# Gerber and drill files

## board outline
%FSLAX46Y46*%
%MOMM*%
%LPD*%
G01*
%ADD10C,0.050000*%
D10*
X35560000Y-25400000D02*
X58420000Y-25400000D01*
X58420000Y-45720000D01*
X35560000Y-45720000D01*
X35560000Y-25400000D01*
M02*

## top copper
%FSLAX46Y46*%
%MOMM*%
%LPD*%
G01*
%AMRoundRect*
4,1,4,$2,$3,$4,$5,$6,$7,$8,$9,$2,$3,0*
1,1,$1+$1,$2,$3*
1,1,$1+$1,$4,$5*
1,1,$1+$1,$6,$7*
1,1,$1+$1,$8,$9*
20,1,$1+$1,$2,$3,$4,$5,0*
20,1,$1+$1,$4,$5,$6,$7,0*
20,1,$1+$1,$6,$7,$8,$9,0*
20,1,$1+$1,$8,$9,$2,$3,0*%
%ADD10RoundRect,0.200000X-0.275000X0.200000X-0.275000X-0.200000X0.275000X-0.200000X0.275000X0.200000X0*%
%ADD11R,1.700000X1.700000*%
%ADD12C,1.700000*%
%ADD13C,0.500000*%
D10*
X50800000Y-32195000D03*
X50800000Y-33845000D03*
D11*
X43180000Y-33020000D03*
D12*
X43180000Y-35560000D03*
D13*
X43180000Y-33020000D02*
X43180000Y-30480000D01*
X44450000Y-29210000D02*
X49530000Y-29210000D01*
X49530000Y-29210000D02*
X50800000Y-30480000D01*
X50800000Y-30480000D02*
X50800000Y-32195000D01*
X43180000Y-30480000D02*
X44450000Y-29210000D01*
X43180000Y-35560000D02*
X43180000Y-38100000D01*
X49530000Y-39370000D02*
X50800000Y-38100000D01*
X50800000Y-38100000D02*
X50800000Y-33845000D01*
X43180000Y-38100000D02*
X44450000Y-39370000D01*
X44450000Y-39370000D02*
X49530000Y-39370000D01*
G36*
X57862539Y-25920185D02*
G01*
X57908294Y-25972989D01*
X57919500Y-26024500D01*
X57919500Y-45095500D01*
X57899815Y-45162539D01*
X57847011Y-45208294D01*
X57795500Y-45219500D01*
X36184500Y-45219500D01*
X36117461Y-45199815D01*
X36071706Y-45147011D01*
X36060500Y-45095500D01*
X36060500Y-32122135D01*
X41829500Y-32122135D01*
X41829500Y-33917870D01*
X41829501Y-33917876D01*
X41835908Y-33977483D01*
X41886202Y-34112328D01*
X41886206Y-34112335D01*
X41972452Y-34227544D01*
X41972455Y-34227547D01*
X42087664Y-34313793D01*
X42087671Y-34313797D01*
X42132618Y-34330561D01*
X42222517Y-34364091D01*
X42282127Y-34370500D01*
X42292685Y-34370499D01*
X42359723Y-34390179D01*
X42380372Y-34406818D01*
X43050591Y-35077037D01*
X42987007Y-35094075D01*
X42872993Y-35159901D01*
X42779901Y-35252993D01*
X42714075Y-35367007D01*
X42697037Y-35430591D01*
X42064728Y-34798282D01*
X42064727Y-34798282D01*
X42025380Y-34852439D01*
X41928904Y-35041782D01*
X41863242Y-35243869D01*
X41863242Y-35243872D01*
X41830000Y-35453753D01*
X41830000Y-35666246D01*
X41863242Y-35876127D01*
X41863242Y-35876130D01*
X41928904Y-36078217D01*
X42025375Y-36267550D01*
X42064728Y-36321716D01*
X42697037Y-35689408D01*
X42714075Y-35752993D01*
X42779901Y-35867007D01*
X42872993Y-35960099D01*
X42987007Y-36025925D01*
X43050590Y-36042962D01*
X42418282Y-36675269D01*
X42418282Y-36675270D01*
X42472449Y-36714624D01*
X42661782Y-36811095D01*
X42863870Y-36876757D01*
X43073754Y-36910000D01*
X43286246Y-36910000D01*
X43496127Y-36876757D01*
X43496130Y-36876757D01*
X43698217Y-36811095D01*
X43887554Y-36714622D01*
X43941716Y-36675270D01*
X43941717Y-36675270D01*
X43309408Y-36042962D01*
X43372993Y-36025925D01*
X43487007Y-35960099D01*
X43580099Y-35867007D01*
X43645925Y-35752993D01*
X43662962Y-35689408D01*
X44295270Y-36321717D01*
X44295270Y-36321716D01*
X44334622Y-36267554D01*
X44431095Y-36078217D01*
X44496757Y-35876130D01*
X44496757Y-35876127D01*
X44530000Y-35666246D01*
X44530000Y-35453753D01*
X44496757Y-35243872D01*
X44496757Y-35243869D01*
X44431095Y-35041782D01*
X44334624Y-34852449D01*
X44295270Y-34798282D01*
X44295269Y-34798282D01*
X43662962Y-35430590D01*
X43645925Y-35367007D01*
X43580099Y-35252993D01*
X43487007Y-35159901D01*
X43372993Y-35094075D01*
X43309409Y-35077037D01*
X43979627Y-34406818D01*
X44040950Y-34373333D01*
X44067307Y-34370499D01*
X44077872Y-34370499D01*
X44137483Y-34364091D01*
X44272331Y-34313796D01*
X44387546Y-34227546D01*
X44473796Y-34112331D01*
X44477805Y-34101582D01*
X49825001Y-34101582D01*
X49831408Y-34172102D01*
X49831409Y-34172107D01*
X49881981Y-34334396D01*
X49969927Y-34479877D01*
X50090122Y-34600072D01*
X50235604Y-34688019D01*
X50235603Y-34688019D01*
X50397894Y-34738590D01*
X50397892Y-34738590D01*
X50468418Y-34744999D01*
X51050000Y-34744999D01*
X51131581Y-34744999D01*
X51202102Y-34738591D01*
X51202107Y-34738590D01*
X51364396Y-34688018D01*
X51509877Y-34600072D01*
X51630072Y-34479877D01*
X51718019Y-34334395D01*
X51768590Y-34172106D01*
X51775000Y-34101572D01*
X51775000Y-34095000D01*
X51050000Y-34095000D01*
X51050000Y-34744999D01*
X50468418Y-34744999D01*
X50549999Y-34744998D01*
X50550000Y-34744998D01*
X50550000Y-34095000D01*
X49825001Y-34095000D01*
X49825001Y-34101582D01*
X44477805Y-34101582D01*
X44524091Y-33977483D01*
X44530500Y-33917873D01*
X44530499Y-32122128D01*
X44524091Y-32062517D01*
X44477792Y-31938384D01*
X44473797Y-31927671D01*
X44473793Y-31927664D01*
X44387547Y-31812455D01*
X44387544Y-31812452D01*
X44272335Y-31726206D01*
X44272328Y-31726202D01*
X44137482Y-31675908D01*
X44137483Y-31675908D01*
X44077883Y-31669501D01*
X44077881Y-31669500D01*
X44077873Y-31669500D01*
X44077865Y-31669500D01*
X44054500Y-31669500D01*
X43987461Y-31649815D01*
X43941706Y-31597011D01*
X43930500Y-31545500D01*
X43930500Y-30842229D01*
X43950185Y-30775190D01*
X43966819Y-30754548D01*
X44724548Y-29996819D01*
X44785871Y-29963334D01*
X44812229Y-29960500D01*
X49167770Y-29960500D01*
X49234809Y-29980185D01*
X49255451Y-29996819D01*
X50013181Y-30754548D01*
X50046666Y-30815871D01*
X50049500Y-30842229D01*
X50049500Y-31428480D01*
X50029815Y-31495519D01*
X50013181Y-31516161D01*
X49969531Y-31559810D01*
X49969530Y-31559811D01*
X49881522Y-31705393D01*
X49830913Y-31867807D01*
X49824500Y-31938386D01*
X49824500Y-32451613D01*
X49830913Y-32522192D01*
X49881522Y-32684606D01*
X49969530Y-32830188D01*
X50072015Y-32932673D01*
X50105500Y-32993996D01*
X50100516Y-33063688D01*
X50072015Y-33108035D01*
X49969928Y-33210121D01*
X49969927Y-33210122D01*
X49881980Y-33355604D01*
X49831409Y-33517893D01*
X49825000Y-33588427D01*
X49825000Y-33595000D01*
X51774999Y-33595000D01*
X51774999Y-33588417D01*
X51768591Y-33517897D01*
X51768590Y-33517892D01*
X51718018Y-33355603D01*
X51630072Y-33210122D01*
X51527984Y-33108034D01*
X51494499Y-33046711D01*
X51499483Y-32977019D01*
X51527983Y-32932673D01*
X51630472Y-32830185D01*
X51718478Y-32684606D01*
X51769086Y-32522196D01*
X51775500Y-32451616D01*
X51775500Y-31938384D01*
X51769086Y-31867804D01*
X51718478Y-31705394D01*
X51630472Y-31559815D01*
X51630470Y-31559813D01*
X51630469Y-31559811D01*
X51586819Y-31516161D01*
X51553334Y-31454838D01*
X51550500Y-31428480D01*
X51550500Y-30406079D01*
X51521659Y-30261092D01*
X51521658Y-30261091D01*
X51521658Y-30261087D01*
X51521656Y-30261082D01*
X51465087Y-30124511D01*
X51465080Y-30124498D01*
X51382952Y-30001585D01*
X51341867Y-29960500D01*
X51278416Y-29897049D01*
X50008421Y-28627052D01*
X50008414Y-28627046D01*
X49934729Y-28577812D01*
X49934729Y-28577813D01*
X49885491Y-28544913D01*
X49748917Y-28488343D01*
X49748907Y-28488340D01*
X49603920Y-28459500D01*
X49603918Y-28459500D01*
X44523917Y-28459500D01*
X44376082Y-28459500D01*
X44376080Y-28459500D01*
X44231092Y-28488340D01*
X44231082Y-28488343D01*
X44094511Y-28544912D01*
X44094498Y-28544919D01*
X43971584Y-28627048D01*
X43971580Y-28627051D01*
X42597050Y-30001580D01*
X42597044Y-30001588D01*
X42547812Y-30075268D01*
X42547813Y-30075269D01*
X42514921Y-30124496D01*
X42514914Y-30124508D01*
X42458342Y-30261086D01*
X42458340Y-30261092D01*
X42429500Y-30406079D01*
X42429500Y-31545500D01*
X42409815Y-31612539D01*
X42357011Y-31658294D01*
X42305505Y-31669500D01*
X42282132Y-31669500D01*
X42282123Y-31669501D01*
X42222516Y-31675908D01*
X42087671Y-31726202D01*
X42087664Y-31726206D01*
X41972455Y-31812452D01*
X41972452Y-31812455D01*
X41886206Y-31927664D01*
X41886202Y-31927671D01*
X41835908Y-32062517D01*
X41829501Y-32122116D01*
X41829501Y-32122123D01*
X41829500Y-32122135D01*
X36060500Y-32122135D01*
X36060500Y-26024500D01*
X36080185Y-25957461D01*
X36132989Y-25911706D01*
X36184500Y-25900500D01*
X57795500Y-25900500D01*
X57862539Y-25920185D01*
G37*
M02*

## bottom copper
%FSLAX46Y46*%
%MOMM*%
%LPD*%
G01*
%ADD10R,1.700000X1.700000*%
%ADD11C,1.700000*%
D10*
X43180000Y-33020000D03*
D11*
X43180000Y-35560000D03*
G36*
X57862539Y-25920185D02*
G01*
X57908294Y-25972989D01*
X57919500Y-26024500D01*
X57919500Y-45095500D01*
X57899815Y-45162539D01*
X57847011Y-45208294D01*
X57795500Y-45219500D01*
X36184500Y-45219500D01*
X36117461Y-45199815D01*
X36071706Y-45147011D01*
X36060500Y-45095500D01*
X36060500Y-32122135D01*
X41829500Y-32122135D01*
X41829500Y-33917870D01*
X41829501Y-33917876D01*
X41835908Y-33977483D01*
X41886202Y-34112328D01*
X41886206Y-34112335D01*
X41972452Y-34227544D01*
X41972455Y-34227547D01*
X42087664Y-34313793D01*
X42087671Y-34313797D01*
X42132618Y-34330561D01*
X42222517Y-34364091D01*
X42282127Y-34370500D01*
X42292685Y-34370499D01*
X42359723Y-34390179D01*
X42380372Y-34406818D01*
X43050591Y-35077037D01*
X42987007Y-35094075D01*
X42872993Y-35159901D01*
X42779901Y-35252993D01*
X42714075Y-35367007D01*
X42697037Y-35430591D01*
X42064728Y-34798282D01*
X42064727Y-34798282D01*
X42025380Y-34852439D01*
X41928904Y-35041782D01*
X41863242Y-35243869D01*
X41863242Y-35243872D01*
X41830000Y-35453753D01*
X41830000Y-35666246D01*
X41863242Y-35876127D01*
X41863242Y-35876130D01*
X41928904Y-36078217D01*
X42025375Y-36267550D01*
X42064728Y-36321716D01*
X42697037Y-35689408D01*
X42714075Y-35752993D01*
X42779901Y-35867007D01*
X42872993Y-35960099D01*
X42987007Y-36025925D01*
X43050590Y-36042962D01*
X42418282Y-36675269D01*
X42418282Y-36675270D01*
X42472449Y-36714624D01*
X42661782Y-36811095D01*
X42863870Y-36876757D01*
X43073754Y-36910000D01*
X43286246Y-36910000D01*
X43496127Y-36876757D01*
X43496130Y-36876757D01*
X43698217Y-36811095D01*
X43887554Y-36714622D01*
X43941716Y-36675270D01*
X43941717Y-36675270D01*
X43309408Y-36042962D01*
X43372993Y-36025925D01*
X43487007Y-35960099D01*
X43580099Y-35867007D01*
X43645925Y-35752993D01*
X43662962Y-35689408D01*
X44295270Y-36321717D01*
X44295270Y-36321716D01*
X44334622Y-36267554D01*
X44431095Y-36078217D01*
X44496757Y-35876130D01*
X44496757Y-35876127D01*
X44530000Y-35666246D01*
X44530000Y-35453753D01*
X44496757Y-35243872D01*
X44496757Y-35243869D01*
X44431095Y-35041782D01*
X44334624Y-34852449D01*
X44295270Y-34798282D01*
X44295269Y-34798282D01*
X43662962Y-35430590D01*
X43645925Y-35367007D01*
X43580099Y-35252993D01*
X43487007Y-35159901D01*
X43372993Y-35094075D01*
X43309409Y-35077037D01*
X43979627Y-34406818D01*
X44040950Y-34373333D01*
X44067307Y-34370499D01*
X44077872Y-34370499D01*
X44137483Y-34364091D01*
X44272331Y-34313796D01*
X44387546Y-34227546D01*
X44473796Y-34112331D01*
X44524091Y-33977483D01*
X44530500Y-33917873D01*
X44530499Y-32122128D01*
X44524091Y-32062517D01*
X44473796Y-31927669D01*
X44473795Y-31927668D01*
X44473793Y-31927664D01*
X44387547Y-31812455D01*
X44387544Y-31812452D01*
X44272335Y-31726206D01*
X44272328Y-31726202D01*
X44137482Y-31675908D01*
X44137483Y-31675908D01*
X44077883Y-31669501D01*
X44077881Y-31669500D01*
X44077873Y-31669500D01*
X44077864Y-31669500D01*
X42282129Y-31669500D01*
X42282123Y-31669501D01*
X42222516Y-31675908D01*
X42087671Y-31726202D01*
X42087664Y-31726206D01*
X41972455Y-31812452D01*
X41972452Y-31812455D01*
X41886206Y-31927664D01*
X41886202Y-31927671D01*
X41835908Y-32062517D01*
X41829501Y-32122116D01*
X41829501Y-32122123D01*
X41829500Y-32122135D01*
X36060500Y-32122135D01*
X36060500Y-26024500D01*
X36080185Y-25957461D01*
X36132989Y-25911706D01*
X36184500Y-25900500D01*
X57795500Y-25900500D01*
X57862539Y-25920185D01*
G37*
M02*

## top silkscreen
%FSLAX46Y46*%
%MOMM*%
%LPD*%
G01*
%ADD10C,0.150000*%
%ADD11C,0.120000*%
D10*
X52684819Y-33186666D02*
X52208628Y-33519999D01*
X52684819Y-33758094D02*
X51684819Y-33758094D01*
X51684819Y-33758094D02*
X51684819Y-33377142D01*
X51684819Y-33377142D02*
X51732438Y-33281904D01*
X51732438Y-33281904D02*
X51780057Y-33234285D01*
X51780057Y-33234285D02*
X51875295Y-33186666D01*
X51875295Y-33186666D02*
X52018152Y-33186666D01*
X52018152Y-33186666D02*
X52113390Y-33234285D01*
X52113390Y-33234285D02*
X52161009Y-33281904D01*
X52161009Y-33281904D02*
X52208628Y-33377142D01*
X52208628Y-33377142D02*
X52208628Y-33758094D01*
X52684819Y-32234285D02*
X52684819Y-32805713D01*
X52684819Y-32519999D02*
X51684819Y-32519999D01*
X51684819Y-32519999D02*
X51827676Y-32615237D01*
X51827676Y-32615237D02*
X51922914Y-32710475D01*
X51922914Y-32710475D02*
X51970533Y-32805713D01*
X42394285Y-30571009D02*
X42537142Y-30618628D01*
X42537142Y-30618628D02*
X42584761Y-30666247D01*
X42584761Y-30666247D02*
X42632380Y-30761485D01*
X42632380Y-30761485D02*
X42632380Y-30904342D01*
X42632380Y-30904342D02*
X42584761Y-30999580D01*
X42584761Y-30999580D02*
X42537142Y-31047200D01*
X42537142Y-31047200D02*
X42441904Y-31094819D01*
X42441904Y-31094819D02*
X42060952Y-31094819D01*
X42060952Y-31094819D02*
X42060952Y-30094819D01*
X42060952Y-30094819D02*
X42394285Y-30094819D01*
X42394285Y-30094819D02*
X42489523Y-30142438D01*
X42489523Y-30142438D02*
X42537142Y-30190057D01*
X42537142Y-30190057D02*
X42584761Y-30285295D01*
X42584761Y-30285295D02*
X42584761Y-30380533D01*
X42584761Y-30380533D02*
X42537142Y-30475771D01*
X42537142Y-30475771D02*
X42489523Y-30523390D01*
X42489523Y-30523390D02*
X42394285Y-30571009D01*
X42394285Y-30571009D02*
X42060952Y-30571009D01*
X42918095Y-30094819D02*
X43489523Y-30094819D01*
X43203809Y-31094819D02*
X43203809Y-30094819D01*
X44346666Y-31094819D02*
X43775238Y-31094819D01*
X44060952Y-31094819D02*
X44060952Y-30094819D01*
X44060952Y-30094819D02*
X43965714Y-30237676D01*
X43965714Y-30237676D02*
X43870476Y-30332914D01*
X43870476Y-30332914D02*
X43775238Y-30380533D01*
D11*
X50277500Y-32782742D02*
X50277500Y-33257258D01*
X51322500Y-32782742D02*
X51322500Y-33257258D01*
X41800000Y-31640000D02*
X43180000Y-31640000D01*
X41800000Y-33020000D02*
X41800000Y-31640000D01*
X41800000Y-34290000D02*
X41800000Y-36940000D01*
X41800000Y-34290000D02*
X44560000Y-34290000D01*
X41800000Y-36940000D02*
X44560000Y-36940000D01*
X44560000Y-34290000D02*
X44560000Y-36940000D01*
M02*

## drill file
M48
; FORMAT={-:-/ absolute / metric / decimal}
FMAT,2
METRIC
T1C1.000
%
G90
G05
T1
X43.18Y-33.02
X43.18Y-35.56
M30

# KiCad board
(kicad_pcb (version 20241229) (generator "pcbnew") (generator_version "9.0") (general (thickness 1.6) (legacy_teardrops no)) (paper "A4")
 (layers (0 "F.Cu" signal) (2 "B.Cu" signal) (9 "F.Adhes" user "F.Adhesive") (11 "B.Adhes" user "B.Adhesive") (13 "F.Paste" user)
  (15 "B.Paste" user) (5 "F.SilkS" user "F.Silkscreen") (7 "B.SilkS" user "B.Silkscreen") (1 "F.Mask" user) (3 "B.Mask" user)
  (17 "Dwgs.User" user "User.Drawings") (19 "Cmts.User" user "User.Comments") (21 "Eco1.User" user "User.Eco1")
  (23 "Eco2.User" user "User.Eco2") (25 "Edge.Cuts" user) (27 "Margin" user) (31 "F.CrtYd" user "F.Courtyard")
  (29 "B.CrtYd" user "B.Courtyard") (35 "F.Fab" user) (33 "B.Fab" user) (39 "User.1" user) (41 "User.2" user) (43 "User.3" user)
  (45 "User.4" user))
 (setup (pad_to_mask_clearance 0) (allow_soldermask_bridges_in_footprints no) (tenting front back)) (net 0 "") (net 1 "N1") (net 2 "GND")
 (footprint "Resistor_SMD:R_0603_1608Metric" (layer "F.Cu") (at 50.8 33.02 -90)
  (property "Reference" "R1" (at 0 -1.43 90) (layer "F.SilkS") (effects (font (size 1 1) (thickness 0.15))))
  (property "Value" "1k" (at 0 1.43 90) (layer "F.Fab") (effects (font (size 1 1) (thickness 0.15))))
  (fp_line (start -0.237258 0.5225) (end 0.237258 0.5225) (stroke (width 0.12) (type solid)) (layer "F.SilkS"))
  (fp_line (start -0.237258 -0.5225) (end 0.237258 -0.5225) (stroke (width 0.12) (type solid)) (layer "F.SilkS"))
  (pad "1" smd roundrect (at -0.825 0 270) (size 0.8 0.95) (layers "F.Cu" "F.Mask" "F.Paste") (roundrect_rratio 0.25) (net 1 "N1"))
  (pad "2" smd roundrect (at 0.825 0 270) (size 0.8 0.95) (layers "F.Cu" "F.Mask" "F.Paste") (roundrect_rratio 0.25) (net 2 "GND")))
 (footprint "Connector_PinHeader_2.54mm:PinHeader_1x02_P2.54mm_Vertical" (layer "F.Cu") (at 43.18 33.02)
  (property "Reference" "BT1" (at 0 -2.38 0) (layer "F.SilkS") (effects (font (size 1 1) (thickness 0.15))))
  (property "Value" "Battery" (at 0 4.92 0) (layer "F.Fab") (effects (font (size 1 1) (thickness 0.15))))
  (fp_line (start -1.38 -1.38) (end 0 -1.38) (stroke (width 0.12) (type solid)) (layer "F.SilkS"))
  (fp_line (start -1.38 0) (end -1.38 -1.38) (stroke (width 0.12) (type solid)) (layer "F.SilkS"))
  (fp_line (start -1.38 1.27) (end -1.38 3.92) (stroke (width 0.12) (type solid)) (layer "F.SilkS"))
  (fp_line (start -1.38 1.27) (end 1.38 1.27) (stroke (width 0.12) (type solid)) (layer "F.SilkS"))
  (fp_line (start -1.38 3.92) (end 1.38 3.92) (stroke (width 0.12) (type solid)) (layer "F.SilkS"))
  (fp_line (start 1.38 1.27) (end 1.38 3.92) (stroke (width 0.12) (type solid)) (layer "F.SilkS"))
  (pad "1" thru_hole rect (at 0 0) (size 1.7 1.7) (drill 1) (layers "*.Cu" "*.Mask") (remove_unused_layers no) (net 1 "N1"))
  (pad "2" thru_hole circle (at 0 2.54) (size 1.7 1.7) (drill 1) (layers "*.Cu" "*.Mask") (remove_unused_layers no) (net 2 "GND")))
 (gr_rect (start 35.56 25.4) (end 58.42 45.72) (stroke (width 0.05) (type default)) (fill no) (layer "Edge.Cuts"))
 (segment (start 43.18 33.02) (end 43.18 30.48) (width 0.5) (layer "F.Cu") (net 1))
 (segment (start 44.45 29.21) (end 49.53 29.21) (width 0.5) (layer "F.Cu") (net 1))
 (segment (start 49.53 29.21) (end 50.8 30.48) (width 0.5) (layer "F.Cu") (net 1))
 (segment (start 50.8 30.48) (end 50.8 32.195) (width 0.5) (layer "F.Cu") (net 1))
 (segment (start 43.18 30.48) (end 44.45 29.21) (width 0.5) (layer "F.Cu") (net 1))
 (segment (start 43.18 35.56) (end 43.18 38.1) (width 0.5) (layer "F.Cu") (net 2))
 (segment (start 49.53 39.37) (end 50.8 38.1) (width 0.5) (layer "F.Cu") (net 2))
 (segment (start 50.8 38.1) (end 50.8 33.845) (width 0.5) (layer "F.Cu") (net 2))
 (segment (start 43.18 38.1) (end 44.45 39.37) (width 0.5) (layer "F.Cu") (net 2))
 (segment (start 44.45 39.37) (end 49.53 39.37) (width 0.5) (layer "F.Cu") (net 2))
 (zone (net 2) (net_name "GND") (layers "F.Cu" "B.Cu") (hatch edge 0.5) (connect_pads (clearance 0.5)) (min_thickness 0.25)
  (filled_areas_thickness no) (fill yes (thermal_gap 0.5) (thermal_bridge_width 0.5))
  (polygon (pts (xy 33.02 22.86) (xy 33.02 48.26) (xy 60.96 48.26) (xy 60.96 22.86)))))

